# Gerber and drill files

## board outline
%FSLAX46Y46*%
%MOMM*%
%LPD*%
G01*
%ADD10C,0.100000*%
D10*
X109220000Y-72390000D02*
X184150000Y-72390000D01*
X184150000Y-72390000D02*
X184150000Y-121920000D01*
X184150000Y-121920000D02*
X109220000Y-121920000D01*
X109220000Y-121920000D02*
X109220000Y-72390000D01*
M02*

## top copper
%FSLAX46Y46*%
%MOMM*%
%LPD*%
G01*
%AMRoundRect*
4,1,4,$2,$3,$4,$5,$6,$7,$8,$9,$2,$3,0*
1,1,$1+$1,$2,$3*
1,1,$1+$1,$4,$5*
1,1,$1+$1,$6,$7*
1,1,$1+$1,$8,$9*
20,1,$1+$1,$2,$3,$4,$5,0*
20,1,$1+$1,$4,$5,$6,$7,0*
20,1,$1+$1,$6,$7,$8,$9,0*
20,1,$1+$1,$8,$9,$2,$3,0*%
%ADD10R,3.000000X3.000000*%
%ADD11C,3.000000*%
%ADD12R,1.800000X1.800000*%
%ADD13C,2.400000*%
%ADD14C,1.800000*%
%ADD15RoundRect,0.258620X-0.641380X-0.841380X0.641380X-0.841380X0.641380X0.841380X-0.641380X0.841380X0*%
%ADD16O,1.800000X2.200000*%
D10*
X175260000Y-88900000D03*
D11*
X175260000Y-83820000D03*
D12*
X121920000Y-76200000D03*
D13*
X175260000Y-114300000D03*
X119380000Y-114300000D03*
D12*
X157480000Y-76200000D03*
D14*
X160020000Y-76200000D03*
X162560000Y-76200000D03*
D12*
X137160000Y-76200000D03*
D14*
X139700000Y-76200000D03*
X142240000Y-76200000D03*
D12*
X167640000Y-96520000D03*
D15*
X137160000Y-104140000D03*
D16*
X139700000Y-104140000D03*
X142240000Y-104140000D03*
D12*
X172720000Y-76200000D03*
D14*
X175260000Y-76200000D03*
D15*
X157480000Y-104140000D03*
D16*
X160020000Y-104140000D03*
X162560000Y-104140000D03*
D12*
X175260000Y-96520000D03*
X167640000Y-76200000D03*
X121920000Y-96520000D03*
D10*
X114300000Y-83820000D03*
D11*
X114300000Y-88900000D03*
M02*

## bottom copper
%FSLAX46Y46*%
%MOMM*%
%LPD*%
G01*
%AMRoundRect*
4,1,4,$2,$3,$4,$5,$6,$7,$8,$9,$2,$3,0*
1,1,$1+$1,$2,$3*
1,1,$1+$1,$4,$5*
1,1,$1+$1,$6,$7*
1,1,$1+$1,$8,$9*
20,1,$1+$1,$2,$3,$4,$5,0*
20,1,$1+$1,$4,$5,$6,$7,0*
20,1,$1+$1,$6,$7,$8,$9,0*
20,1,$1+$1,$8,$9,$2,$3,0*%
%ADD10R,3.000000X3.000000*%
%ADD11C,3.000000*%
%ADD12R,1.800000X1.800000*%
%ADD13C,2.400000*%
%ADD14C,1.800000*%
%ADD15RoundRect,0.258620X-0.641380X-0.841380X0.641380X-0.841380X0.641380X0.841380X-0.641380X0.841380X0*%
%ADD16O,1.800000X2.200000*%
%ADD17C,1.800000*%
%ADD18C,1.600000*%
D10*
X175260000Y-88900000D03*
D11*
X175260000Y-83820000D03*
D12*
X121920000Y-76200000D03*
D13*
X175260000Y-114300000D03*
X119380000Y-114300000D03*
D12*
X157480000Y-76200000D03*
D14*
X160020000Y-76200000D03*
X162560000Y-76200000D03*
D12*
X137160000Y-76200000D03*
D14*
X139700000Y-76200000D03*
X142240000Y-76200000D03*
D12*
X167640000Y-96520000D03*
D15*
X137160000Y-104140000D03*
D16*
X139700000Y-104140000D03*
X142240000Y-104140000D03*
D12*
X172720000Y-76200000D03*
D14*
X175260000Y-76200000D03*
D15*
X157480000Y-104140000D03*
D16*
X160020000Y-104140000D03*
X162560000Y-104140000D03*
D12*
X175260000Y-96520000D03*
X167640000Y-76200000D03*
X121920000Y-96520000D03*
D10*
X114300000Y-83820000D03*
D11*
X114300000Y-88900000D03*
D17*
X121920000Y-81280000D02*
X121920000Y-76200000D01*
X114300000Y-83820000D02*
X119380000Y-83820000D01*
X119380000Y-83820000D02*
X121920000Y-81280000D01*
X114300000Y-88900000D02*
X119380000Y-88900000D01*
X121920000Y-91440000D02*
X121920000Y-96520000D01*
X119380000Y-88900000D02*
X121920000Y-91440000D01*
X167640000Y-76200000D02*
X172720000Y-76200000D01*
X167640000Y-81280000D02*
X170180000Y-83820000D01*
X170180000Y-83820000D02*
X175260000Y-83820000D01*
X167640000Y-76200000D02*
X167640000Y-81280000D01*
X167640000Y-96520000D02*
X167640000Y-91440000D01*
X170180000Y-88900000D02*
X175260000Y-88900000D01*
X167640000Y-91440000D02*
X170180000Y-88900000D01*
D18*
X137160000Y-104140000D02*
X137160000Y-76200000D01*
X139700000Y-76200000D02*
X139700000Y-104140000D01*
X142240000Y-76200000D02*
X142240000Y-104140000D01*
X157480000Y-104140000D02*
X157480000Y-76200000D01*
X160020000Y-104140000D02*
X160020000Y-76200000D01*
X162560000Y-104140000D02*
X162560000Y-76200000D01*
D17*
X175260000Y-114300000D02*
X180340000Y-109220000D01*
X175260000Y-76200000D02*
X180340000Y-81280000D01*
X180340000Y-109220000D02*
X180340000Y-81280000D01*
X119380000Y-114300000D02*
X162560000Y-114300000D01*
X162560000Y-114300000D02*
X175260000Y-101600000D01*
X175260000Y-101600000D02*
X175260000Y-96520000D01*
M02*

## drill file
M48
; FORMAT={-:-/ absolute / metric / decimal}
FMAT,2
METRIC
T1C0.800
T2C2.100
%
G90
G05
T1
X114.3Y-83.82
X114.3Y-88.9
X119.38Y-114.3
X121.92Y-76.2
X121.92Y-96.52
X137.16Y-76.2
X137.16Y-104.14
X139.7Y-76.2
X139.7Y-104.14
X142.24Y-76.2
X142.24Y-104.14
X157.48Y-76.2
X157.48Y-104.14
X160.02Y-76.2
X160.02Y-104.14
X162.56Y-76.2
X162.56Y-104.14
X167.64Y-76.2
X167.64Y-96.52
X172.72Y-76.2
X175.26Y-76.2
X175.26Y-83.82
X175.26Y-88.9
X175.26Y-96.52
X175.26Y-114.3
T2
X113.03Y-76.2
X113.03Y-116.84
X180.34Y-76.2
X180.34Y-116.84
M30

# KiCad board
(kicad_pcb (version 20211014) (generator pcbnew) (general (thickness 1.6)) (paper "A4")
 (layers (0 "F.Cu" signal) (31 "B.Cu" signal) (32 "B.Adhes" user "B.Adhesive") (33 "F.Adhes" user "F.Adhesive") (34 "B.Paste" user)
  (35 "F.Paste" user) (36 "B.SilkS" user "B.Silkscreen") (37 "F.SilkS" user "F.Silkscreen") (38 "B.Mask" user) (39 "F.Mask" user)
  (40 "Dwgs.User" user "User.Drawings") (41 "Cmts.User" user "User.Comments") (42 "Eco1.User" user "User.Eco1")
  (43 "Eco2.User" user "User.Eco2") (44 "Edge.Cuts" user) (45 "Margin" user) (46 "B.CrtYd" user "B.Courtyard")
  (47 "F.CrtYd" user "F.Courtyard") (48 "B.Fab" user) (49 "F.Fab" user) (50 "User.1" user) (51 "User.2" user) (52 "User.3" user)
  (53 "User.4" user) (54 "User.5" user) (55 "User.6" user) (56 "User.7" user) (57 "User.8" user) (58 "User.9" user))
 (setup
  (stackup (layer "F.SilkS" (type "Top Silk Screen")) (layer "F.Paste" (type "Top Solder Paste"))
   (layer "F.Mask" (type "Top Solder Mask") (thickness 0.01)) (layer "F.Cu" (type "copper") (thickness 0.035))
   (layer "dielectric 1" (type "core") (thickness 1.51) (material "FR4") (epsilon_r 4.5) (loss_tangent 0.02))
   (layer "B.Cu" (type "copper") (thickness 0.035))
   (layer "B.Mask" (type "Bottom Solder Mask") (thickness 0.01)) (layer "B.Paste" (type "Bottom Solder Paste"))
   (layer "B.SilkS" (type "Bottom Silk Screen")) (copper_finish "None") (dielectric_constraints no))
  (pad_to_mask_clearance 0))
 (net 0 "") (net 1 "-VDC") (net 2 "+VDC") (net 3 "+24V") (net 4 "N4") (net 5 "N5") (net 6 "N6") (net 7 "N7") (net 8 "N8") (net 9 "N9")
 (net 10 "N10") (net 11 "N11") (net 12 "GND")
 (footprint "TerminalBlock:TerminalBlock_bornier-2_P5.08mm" (layer "F.Cu") (at 175.26 88.9 90)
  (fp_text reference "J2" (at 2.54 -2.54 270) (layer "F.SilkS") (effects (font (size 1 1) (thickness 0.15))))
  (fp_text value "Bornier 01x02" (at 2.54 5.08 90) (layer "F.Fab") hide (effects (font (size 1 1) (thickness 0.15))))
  (pad "1" thru_hole rect (at 0 0 90) (size 3 3) (drill 0.8) (layers *.Cu *.Mask) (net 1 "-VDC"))
  (pad "2" thru_hole circle (at 5.08 0 90) (size 3 3) (drill 0.8) (layers *.Cu *.Mask) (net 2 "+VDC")))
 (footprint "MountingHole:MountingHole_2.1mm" (layer "F.Cu") (at 180.34 116.84)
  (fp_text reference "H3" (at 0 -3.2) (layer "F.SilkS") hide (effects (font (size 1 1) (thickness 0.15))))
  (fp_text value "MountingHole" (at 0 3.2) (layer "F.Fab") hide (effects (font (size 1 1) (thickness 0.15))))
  (pad "" np_thru_hole circle (at 0 0) (size 2.1 2.1) (drill 2.1) (layers *.Cu *.Mask)))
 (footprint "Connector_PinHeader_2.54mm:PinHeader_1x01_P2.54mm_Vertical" (layer "F.Cu") (at 121.92 76.2)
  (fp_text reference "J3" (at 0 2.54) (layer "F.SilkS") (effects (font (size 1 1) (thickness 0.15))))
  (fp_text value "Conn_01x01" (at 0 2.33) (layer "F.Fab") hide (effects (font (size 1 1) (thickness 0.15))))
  (pad "1" thru_hole rect (at 0 0) (size 1.8 1.8) (drill 0.8) (layers *.Cu *.Mask) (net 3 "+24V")))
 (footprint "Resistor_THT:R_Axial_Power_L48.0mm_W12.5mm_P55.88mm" (layer "F.Cu") (at 175.26 114.3 180)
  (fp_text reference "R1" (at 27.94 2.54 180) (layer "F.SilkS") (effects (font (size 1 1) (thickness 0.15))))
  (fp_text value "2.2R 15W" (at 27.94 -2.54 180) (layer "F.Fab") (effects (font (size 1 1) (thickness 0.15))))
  (pad "1" thru_hole circle (at 0 0 180) (size 2.4 2.4) (drill 0.8) (layers *.Cu *.Mask) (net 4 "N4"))
  (pad "2" thru_hole circle (at 55.88 0 180) (size 2.4 2.4) (drill 0.8) (layers *.Cu *.Mask) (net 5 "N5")))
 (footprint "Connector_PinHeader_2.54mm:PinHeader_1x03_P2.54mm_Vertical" (layer "F.Cu") (at 157.48 76.2 90)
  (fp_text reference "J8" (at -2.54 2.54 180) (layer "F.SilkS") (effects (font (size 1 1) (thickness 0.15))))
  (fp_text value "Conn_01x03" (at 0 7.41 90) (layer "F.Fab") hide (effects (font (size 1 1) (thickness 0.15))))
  (pad "1" thru_hole rect (at 0 0 90) (size 1.8 1.8) (drill 0.8) (layers *.Cu *.Mask) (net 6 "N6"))
  (pad "2" thru_hole circle (at 0 2.54 90) (size 1.8 1.8) (drill 0.8) (layers *.Cu *.Mask) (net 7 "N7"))
  (pad "3" thru_hole circle (at 0 5.08 90) (size 1.8 1.8) (drill 0.8) (layers *.Cu *.Mask) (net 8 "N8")))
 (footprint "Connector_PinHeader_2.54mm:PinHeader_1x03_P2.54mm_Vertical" (layer "F.Cu") (at 137.16 76.2 90)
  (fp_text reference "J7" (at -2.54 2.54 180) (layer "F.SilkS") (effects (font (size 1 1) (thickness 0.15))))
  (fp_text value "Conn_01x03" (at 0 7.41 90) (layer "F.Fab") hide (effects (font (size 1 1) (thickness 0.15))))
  (pad "1" thru_hole rect (at 0 0 90) (size 1.8 1.8) (drill 0.8) (layers *.Cu *.Mask) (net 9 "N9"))
  (pad "2" thru_hole circle (at 0 2.54 90) (size 1.8 1.8) (drill 0.8) (layers *.Cu *.Mask) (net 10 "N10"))
  (pad "3" thru_hole circle (at 0 5.08 90) (size 1.8 1.8) (drill 0.8) (layers *.Cu *.Mask) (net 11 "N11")))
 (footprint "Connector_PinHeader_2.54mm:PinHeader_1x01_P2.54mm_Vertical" (layer "F.Cu") (at 167.64 96.52)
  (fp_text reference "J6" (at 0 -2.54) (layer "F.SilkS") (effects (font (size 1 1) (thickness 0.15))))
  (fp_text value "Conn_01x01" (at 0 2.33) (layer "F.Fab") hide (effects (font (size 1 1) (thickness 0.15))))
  (pad "1" thru_hole rect (at 0 0) (size 1.8 1.8) (drill 0.8) (layers *.Cu *.Mask) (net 1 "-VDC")))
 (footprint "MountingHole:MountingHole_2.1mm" (layer "F.Cu") (at 113.03 116.84)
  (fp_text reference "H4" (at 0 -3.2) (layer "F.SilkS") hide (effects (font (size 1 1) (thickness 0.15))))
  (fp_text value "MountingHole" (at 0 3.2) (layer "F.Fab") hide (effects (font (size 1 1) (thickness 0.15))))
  (pad "" np_thru_hole circle (at 0 0) (size 2.1 2.1) (drill 2.1) (layers *.Cu *.Mask)))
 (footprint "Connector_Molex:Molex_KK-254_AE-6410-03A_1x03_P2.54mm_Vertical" (layer "F.Cu") (at 137.16 104.14)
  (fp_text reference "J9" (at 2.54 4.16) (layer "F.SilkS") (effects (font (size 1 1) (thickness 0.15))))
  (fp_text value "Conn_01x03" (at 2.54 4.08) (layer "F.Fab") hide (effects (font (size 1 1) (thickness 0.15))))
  (pad "1" thru_hole roundrect (at 0 0) (size 1.8 2.2) (drill 0.8) (layers *.Cu *.Mask) (roundrect_rratio 0.143678) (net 9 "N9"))
  (pad "2" thru_hole oval (at 2.54 0) (size 1.8 2.2) (drill 0.8) (layers *.Cu *.Mask) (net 10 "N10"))
  (pad "3" thru_hole oval (at 5.08 0) (size 1.8 2.2) (drill 0.8) (layers *.Cu *.Mask) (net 11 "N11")))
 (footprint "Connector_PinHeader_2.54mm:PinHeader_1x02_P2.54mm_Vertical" (layer "F.Cu") (at 172.72 76.2 90)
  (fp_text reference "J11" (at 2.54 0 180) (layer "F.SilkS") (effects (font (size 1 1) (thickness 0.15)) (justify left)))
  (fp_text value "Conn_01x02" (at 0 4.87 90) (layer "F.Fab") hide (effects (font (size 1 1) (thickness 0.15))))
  (pad "1" thru_hole rect (at 0 0 90) (size 1.8 1.8) (drill 0.8) (layers *.Cu *.Mask) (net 2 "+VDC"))
  (pad "2" thru_hole circle (at 0 2.54 90) (size 1.8 1.8) (drill 0.8) (layers *.Cu *.Mask) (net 4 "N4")))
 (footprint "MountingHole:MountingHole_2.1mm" (layer "F.Cu") (at 180.34 76.2)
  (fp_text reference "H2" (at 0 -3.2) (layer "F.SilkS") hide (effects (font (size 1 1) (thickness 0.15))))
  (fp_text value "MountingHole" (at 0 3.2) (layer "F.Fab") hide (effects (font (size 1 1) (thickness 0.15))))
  (pad "" np_thru_hole circle (at 0 0) (size 2.1 2.1) (drill 2.1) (layers *.Cu *.Mask)))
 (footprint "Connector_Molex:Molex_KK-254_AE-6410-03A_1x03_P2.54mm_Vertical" (layer "F.Cu") (at 157.48 104.14)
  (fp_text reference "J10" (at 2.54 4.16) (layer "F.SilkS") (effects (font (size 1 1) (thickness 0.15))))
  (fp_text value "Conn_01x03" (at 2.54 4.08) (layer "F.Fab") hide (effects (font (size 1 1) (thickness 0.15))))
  (pad "1" thru_hole roundrect (at 0 0) (size 1.8 2.2) (drill 0.8) (layers *.Cu *.Mask) (roundrect_rratio 0.143678) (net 6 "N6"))
  (pad "2" thru_hole oval (at 2.54 0) (size 1.8 2.2) (drill 0.8) (layers *.Cu *.Mask) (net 7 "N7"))
  (pad "3" thru_hole oval (at 5.08 0) (size 1.8 2.2) (drill 0.8) (layers *.Cu *.Mask) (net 8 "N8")))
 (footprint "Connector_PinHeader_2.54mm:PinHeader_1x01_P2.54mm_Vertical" (layer "F.Cu") (at 175.26 96.52)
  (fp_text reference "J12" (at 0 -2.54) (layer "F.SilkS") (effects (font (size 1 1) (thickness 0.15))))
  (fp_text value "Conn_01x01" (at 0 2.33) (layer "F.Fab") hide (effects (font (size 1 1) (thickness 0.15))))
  (pad "1" thru_hole rect (at 0 0) (size 1.8 1.8) (drill 0.8) (layers *.Cu *.Mask) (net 5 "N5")))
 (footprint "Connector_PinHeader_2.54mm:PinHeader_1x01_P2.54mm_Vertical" (layer "F.Cu") (at 167.64 76.2)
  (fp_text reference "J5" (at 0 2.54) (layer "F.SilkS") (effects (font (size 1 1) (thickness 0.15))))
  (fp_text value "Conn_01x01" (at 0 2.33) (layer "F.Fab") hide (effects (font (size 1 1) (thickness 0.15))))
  (pad "1" thru_hole rect (at 0 0) (size 1.8 1.8) (drill 0.8) (layers *.Cu *.Mask) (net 2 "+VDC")))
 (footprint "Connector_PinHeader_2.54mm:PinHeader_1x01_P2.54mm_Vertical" (layer "F.Cu") (at 121.92 96.52)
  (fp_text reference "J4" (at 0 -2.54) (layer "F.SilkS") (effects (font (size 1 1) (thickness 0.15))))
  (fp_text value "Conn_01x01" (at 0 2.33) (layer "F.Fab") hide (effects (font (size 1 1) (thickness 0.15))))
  (pad "1" thru_hole rect (at 0 0) (size 1.8 1.8) (drill 0.8) (layers *.Cu *.Mask) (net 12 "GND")))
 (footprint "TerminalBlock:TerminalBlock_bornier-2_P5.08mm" (layer "F.Cu") (at 114.3 83.82 -90)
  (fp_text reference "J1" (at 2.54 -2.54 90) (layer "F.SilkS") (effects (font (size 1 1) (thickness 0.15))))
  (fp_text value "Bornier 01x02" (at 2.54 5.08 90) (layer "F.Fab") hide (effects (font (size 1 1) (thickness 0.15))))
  (pad "1" thru_hole rect (at 0 0 270) (size 3 3) (drill 0.8) (layers *.Cu *.Mask) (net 3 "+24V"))
  (pad "2" thru_hole circle (at 5.08 0 270) (size 3 3) (drill 0.8) (layers *.Cu *.Mask) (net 12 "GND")))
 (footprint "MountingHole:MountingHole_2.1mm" (layer "F.Cu") (at 113.03 76.2)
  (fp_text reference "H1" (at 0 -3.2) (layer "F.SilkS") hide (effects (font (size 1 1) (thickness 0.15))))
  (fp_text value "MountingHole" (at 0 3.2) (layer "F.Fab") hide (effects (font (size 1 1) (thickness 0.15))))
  (pad "" np_thru_hole circle (at 0 0) (size 2.1 2.1) (drill 2.1) (layers *.Cu *.Mask)))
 (gr_line (start 109.22 72.39) (end 184.15 72.39) (layer "Edge.Cuts") (width 0.1))
 (gr_line (start 184.15 72.39) (end 184.15 121.92) (layer "Edge.Cuts") (width 0.1))
 (gr_line (start 184.15 121.92) (end 109.22 121.92) (layer "Edge.Cuts") (width 0.1))
 (gr_line (start 109.22 121.92) (end 109.22 72.39) (layer "Edge.Cuts") (width 0.1))
 (segment (start 121.92 81.28) (end 121.92 76.2) (width 1.8) (layer "B.Cu") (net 3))
 (segment (start 114.3 83.82) (end 119.38 83.82) (width 1.8) (layer "B.Cu") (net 3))
 (segment (start 119.38 83.82) (end 121.92 81.28) (width 1.8) (layer "B.Cu") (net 3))
 (segment (start 114.3 88.9) (end 119.38 88.9) (width 1.8) (layer "B.Cu") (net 12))
 (segment (start 121.92 91.44) (end 121.92 96.52) (width 1.8) (layer "B.Cu") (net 12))
 (segment (start 119.38 88.9) (end 121.92 91.44) (width 1.8) (layer "B.Cu") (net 12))
 (segment (start 167.64 76.2) (end 172.72 76.2) (width 1.8) (layer "B.Cu") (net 2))
 (segment (start 167.64 81.28) (end 170.18 83.82) (width 1.8) (layer "B.Cu") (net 2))
 (segment (start 170.18 83.82) (end 175.26 83.82) (width 1.8) (layer "B.Cu") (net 2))
 (segment (start 167.64 76.2) (end 167.64 81.28) (width 1.8) (layer "B.Cu") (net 2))
 (segment (start 167.64 96.52) (end 167.64 91.44) (width 1.8) (layer "B.Cu") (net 1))
 (segment (start 170.18 88.9) (end 175.26 88.9) (width 1.8) (layer "B.Cu") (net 1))
 (segment (start 167.64 91.44) (end 170.18 88.9) (width 1.8) (layer "B.Cu") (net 1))
 (segment (start 137.16 104.14) (end 137.16 76.2) (width 1.6) (layer "B.Cu") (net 9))
 (segment (start 139.7 76.2) (end 139.7 104.14) (width 1.6) (layer "B.Cu") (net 10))
 (segment (start 142.24 76.2) (end 142.24 104.14) (width 1.6) (layer "B.Cu") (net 11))
 (segment (start 157.48 104.14) (end 157.48 76.2) (width 1.6) (layer "B.Cu") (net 6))
 (segment (start 160.02 104.14) (end 160.02 76.2) (width 1.6) (layer "B.Cu") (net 7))
 (segment (start 162.56 104.14) (end 162.56 76.2) (width 1.6) (layer "B.Cu") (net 8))
 (segment (start 175.26 114.3) (end 180.34 109.22) (width 1.8) (layer "B.Cu") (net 4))
 (segment (start 175.26 76.2) (end 180.34 81.28) (width 1.8) (layer "B.Cu") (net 4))
 (segment (start 180.34 109.22) (end 180.34 81.28) (width 1.8) (layer "B.Cu") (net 4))
 (segment (start 119.38 114.3) (end 162.56 114.3) (width 1.8) (layer "B.Cu") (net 5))
 (segment (start 162.56 114.3) (end 175.26 101.6) (width 1.8) (layer "B.Cu") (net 5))
 (segment (start 175.26 101.6) (end 175.26 96.52) (width 1.8) (layer "B.Cu") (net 5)))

